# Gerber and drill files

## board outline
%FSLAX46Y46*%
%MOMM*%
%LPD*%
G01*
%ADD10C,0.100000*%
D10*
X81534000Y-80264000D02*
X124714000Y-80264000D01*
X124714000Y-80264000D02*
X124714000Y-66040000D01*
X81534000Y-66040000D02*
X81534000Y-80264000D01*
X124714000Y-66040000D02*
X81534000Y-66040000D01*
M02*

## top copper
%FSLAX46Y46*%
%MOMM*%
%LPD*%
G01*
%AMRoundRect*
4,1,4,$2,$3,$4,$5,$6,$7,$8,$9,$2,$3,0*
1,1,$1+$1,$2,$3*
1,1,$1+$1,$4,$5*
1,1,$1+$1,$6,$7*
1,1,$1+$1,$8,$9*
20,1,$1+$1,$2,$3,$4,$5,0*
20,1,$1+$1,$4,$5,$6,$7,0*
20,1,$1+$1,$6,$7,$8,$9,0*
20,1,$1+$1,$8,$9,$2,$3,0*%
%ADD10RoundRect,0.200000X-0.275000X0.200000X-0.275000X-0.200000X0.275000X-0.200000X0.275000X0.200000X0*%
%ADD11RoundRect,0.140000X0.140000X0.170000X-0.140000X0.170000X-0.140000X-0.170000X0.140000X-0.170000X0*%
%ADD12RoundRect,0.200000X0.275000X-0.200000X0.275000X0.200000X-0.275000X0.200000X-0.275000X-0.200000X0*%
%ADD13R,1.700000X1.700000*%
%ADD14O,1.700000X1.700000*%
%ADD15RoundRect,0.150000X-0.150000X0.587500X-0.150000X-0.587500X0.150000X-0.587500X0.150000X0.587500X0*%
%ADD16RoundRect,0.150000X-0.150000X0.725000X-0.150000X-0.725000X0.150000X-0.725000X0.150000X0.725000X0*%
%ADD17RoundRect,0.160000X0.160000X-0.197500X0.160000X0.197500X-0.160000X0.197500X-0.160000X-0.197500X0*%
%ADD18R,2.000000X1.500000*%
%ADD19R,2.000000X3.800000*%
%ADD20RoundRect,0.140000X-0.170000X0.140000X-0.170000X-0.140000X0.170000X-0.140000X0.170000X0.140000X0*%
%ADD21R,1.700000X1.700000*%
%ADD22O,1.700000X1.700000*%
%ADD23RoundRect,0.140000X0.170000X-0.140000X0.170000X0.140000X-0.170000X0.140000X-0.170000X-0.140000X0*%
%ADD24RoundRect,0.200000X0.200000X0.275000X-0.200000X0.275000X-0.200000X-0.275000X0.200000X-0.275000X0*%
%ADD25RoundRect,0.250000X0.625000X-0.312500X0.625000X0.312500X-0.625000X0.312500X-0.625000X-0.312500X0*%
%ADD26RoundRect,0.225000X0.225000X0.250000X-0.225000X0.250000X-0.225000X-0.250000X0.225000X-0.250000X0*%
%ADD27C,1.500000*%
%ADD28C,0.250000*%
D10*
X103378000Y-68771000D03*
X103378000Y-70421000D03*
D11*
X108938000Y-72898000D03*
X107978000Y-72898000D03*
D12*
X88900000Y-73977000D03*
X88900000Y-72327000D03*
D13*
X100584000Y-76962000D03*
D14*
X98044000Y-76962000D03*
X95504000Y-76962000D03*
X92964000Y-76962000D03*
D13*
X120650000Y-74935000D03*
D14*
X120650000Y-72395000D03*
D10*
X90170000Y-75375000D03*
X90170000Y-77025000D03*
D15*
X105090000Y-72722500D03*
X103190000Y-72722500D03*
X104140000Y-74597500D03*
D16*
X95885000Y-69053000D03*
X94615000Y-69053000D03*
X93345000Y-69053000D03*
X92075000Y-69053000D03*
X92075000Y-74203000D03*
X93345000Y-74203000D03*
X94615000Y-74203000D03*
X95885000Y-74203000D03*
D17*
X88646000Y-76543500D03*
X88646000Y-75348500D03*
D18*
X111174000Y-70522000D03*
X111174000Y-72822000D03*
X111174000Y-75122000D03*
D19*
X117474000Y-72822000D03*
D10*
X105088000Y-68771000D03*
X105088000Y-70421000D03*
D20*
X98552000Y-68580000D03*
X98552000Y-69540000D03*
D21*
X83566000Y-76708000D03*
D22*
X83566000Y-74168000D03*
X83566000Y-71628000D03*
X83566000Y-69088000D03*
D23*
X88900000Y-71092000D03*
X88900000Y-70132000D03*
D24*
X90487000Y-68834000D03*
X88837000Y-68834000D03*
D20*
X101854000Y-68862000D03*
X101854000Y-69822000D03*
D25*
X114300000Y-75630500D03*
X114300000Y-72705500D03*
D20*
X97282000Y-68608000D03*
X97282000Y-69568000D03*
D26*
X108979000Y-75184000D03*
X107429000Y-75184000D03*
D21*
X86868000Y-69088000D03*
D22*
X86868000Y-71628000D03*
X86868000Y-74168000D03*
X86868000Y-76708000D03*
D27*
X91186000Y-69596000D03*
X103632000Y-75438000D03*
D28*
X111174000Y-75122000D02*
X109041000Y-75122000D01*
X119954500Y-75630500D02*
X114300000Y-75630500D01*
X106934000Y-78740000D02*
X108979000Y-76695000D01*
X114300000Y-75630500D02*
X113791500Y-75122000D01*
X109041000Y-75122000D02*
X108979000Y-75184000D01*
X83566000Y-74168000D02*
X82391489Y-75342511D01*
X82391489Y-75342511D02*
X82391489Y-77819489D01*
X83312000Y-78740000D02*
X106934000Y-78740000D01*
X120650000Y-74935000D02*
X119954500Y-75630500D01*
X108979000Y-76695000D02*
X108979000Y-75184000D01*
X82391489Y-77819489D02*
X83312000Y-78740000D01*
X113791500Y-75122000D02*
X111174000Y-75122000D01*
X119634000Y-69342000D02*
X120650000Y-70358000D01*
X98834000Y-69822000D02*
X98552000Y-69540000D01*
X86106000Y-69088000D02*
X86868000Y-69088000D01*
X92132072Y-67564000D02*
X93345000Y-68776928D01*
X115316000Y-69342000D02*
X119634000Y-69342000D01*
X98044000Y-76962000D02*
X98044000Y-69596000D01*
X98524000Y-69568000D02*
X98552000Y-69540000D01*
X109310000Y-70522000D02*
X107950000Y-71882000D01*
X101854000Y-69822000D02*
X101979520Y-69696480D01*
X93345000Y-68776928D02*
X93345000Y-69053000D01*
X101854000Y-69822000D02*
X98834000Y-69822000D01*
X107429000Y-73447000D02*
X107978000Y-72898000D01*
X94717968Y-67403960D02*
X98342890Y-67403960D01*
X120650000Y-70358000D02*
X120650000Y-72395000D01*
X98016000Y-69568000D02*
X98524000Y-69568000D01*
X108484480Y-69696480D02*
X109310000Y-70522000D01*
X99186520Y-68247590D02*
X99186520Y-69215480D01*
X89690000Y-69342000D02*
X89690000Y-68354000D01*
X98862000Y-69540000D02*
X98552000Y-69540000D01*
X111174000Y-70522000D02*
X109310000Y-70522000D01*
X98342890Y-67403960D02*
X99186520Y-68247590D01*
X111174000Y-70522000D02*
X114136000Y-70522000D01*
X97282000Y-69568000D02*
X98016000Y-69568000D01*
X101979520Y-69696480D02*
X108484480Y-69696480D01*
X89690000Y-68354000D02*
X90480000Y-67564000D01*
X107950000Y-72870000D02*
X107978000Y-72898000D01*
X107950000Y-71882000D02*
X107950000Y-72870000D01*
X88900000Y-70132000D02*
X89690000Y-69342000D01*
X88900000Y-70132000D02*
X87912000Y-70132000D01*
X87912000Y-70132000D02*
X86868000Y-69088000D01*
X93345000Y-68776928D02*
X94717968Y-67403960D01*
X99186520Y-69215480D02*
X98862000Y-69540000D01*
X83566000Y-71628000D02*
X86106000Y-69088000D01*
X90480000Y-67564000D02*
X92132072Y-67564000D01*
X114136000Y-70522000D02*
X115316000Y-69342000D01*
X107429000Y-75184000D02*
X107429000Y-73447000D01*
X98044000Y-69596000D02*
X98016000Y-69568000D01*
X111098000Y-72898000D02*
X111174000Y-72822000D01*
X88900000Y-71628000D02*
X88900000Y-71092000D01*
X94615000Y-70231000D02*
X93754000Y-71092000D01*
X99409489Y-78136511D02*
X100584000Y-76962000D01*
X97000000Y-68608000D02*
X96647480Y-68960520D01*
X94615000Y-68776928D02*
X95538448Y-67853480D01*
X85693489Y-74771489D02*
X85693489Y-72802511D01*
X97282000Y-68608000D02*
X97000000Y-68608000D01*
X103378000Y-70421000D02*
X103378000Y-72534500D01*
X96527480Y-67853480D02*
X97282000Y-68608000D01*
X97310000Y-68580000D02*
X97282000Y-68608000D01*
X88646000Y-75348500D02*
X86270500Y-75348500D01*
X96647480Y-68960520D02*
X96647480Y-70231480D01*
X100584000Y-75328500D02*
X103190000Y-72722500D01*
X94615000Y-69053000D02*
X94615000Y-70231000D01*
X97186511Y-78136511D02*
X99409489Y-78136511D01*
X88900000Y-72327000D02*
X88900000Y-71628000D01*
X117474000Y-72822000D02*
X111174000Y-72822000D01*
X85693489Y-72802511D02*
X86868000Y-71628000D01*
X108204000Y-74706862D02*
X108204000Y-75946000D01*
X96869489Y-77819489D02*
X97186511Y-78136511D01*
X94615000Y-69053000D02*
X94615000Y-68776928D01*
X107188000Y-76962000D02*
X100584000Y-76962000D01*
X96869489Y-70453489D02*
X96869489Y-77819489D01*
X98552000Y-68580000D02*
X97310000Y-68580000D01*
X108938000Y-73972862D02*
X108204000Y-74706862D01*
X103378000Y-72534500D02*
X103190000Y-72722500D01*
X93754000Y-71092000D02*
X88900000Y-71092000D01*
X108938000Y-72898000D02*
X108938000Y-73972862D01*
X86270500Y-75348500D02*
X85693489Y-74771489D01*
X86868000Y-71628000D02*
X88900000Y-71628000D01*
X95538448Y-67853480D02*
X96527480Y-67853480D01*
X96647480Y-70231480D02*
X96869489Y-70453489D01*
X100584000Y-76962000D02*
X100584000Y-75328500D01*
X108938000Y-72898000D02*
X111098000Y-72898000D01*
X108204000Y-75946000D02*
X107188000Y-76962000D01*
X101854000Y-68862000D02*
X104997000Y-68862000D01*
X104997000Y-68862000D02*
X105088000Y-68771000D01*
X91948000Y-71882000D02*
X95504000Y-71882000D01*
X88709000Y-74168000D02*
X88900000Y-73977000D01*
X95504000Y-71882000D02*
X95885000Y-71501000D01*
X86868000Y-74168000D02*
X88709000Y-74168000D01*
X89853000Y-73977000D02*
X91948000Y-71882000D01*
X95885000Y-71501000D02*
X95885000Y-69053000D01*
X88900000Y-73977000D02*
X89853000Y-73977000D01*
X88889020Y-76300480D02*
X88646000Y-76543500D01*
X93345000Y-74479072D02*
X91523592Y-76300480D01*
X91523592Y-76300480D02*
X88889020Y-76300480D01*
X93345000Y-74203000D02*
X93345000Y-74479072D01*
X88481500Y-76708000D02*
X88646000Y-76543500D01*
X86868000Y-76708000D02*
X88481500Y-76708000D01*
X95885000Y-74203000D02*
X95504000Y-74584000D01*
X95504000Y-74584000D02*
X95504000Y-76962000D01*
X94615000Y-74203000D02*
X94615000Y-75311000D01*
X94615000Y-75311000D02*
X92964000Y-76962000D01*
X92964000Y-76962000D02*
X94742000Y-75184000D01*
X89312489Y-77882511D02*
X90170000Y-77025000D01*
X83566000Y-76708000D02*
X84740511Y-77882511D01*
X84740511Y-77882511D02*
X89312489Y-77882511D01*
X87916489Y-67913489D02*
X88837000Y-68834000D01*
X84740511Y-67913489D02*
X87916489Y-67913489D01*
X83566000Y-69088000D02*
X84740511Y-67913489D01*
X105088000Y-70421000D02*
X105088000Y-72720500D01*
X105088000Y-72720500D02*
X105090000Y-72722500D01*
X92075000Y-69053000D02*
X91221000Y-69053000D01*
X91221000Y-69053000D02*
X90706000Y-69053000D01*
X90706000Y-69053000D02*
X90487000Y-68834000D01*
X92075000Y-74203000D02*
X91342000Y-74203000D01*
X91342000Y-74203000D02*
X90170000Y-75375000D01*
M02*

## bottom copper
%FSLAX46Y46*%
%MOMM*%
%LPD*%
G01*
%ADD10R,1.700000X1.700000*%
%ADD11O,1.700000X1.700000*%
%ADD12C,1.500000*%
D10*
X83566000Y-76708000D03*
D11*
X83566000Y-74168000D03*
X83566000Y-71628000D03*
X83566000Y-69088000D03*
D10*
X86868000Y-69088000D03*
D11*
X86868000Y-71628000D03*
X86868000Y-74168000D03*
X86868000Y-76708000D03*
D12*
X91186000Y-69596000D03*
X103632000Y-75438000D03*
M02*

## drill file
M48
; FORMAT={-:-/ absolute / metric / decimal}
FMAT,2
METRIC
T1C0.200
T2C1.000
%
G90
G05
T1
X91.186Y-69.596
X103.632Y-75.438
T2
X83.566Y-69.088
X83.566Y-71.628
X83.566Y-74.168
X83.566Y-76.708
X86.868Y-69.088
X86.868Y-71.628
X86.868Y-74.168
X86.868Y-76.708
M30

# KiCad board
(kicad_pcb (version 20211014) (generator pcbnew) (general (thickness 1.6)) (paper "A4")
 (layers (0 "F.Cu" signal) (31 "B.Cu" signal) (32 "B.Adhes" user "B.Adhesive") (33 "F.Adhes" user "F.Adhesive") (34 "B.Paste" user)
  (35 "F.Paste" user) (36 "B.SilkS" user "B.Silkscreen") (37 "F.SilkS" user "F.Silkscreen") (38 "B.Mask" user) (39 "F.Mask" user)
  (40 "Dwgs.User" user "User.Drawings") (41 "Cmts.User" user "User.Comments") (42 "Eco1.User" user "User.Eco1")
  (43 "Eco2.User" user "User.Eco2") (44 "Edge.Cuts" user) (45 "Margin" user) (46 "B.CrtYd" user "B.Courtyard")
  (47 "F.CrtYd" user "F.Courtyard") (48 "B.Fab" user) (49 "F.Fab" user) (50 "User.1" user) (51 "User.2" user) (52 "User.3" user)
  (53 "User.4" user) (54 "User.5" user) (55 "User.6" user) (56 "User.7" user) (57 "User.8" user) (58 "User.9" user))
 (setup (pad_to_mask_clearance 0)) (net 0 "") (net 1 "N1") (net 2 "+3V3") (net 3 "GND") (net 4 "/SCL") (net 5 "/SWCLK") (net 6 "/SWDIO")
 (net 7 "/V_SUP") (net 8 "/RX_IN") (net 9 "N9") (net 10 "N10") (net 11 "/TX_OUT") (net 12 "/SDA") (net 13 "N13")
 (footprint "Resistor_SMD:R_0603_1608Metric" (layer "F.Cu") (at 103.378 69.596 -90)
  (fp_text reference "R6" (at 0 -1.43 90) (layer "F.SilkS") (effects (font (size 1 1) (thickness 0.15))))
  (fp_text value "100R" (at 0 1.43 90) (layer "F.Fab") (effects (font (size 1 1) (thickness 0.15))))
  (pad "1" smd roundrect locked (at -0.825 0 270) (size 0.8 0.95) (layers "F.Cu" "F.Paste" "F.Mask") (roundrect_rratio 0.25) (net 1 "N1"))
  (pad "2" smd roundrect locked (at 0.825 0 270) (size 0.8 0.95) (layers "F.Cu" "F.Paste" "F.Mask") (roundrect_rratio 0.25) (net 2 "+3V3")))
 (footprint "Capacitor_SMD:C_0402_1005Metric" (layer "F.Cu") (at 108.458 72.898 180)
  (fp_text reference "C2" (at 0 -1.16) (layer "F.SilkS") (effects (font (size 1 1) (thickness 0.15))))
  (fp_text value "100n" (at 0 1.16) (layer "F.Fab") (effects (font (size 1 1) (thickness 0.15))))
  (pad "1" smd roundrect locked (at -0.48 0 180) (size 0.56 0.62) (layers "F.Cu" "F.Paste" "F.Mask") (roundrect_rratio 0.25) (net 2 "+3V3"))
  (pad "2" smd roundrect locked (at 0.48 0 180) (size 0.56 0.62) (layers "F.Cu" "F.Paste" "F.Mask") (roundrect_rratio 0.25) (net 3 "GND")))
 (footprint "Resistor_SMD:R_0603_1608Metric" (layer "F.Cu") (at 88.9 73.152 90)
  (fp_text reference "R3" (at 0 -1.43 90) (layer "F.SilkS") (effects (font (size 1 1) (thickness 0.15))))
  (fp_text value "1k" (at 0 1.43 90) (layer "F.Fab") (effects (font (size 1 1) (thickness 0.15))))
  (pad "1" smd roundrect locked (at -0.825 0 90) (size 0.8 0.95) (layers "F.Cu" "F.Paste" "F.Mask") (roundrect_rratio 0.25) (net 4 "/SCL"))
  (pad "2" smd roundrect locked (at 0.825 0 90) (size 0.8 0.95) (layers "F.Cu" "F.Paste" "F.Mask") (roundrect_rratio 0.25) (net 2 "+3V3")))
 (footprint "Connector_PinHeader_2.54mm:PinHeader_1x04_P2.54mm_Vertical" (layer "F.Cu") (at 100.584 76.962 -90)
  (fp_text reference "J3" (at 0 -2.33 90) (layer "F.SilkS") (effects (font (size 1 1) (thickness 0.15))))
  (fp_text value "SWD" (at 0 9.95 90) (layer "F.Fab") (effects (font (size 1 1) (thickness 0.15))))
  (pad "1" smd rect locked (at 0 0 270) (size 1.7 1.7) (layers "F.Cu" "F.Paste" "F.Mask") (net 2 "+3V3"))
  (pad "2" smd oval locked (at 0 2.54 270) (size 1.7 1.7) (layers "F.Cu" "F.Paste" "F.Mask") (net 3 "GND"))
  (pad "3" smd oval locked (at 0 5.08 270) (size 1.7 1.7) (layers "F.Cu" "F.Paste" "F.Mask") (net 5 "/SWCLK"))
  (pad "4" smd oval locked (at 0 7.62 270) (size 1.7 1.7) (layers "F.Cu" "F.Paste" "F.Mask") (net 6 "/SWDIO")))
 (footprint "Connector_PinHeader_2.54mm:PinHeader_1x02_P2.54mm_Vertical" (layer "F.Cu") (at 120.65 74.935 180)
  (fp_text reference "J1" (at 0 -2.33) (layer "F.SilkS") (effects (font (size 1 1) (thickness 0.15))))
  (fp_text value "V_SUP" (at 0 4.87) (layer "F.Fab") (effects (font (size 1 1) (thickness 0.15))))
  (pad "1" smd rect locked (at 0 0 180) (size 1.7 1.7) (layers "F.Cu" "F.Paste" "F.Mask") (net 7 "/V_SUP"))
  (pad "2" smd oval locked (at 0 2.54 180) (size 1.7 1.7) (layers "F.Cu" "F.Paste" "F.Mask") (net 3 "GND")))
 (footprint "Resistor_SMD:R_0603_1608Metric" (layer "F.Cu") (at 90.17 76.2 -90)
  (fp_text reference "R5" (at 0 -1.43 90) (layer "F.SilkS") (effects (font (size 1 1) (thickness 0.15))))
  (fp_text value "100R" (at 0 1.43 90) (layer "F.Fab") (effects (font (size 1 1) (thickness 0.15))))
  (pad "1" smd roundrect locked (at -0.825 0 270) (size 0.8 0.95) (layers "F.Cu" "F.Paste" "F.Mask") (roundrect_rratio 0.25)
   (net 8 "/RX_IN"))
  (pad "2" smd roundrect locked (at 0.825 0 270) (size 0.8 0.95) (layers "F.Cu" "F.Paste" "F.Mask") (roundrect_rratio 0.25) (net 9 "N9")))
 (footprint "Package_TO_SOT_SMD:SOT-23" (layer "F.Cu") (at 104.14 73.66 -90)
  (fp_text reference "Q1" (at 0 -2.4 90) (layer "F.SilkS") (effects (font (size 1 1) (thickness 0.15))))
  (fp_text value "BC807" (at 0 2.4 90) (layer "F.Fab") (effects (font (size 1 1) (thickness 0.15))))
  (pad "1" smd roundrect locked (at -0.9375 -0.95 270) (size 1.475 0.6) (layers "F.Cu" "F.Paste" "F.Mask") (roundrect_rratio 0.25)
   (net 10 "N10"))
  (pad "2" smd roundrect locked (at -0.9375 0.95 270) (size 1.475 0.6) (layers "F.Cu" "F.Paste" "F.Mask") (roundrect_rratio 0.25)
   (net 2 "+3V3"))
  (pad "3" smd roundrect locked (at 0.9375 0 270) (size 1.475 0.6) (layers "F.Cu" "F.Paste" "F.Mask") (roundrect_rratio 0.25)
   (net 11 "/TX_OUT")))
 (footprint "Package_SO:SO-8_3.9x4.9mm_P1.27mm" (layer "F.Cu") (at 93.98 71.628 -90)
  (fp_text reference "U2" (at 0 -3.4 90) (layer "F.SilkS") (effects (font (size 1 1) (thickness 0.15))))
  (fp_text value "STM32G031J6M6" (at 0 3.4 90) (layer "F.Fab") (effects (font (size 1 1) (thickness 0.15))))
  (pad "1" smd roundrect locked (at -2.575 -1.905 270) (size 1.75 0.6) (layers "F.Cu" "F.Paste" "F.Mask") (roundrect_rratio 0.25)
   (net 4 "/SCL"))
  (pad "2" smd roundrect locked (at -2.575 -0.635 270) (size 1.75 0.6) (layers "F.Cu" "F.Paste" "F.Mask") (roundrect_rratio 0.25)
   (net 2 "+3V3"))
  (pad "3" smd roundrect locked (at -2.575 0.635 270) (size 1.75 0.6) (layers "F.Cu" "F.Paste" "F.Mask") (roundrect_rratio 0.25)
   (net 3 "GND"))
  (pad "4" smd roundrect locked (at -2.575 1.905 270) (size 1.75 0.6) (layers "F.Cu" "F.Paste" "F.Mask") (roundrect_rratio 0.25)
   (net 11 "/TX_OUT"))
  (pad "5" smd roundrect locked (at 2.575 1.905 270) (size 1.75 0.6) (layers "F.Cu" "F.Paste" "F.Mask") (roundrect_rratio 0.25)
   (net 8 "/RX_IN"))
  (pad "6" smd roundrect locked (at 2.575 0.635 270) (size 1.75 0.6) (layers "F.Cu" "F.Paste" "F.Mask") (roundrect_rratio 0.25)
   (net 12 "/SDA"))
  (pad "7" smd roundrect locked (at 2.575 -0.635 270) (size 1.75 0.6) (layers "F.Cu" "F.Paste" "F.Mask") (roundrect_rratio 0.25)
   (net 6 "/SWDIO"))
  (pad "8" smd roundrect locked (at 2.575 -1.905 270) (size 1.75 0.6) (layers "F.Cu" "F.Paste" "F.Mask") (roundrect_rratio 0.25)
   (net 5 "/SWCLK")))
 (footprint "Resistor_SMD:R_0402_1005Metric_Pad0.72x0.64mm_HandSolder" (layer "F.Cu") (at 88.646 75.946 90)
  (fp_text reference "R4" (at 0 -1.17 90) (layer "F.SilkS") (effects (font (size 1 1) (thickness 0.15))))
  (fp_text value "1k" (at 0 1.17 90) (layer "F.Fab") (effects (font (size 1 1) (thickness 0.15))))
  (pad "1" smd roundrect locked (at -0.5975 0 90) (size 0.715 0.64) (layers "F.Cu" "F.Paste" "F.Mask") (roundrect_rratio 0.25)
   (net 12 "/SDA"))
  (pad "2" smd roundrect locked (at 0.5975 0 90) (size 0.715 0.64) (layers "F.Cu" "F.Paste" "F.Mask") (roundrect_rratio 0.25) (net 2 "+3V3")))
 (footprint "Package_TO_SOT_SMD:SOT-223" (layer "F.Cu") (at 114.324 72.822)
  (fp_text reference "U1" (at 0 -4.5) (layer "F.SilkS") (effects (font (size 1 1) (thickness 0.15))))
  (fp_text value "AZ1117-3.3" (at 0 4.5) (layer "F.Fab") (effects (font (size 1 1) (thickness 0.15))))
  (pad "1" smd rect locked (at -3.15 -2.3) (size 2 1.5) (layers "F.Cu" "F.Paste" "F.Mask") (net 3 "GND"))
  (pad "2" smd rect locked (at -3.15 0) (size 2 1.5) (layers "F.Cu" "F.Paste" "F.Mask") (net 2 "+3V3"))
  (pad "3" smd rect locked (at -3.15 2.3) (size 2 1.5) (layers "F.Cu" "F.Paste" "F.Mask") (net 7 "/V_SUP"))
  (pad "4" smd rect locked (at 3.15 0) (size 2 3.8) (layers "F.Cu" "F.Paste" "F.Mask") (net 2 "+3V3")))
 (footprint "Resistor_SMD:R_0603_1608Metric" (layer "F.Cu") (at 105.088 69.596 -90)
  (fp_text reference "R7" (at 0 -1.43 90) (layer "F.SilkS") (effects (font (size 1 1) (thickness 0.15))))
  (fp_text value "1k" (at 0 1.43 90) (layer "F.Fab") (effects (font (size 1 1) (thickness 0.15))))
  (pad "1" smd roundrect locked (at -0.825 0 270) (size 0.8 0.95) (layers "F.Cu" "F.Paste" "F.Mask") (roundrect_rratio 0.25) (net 1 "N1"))
  (pad "2" smd roundrect locked (at 0.825 0 270) (size 0.8 0.95) (layers "F.Cu" "F.Paste" "F.Mask") (roundrect_rratio 0.25) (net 10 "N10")))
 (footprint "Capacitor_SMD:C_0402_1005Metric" (layer "F.Cu") (at 98.552 69.06 -90)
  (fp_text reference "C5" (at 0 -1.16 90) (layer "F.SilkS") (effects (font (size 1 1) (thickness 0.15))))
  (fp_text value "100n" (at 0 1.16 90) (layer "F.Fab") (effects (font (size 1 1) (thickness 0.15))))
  (pad "1" smd roundrect locked (at -0.48 0 270) (size 0.56 0.62) (layers "F.Cu" "F.Paste" "F.Mask") (roundrect_rratio 0.25) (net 2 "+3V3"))
  (pad "2" smd roundrect locked (at 0.48 0 270) (size 0.56 0.62) (layers "F.Cu" "F.Paste" "F.Mask") (roundrect_rratio 0.25) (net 3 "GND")))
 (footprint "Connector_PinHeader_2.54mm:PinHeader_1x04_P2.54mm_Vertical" (layer "F.Cu") (at 83.566 76.708 180)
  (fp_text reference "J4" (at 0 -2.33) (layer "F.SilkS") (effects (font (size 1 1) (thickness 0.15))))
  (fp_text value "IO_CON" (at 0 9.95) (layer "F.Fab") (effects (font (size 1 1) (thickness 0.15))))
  (pad "1" thru_hole rect locked (at 0 0 180) (size 1.7 1.7) (drill 1) (layers *.Cu *.Mask) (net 9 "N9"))
  (pad "2" thru_hole oval locked (at 0 2.54 180) (size 1.7 1.7) (drill 1) (layers *.Cu *.Mask) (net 7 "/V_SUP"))
  (pad "3" thru_hole oval locked (at 0 5.08 180) (size 1.7 1.7) (drill 1) (layers *.Cu *.Mask) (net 3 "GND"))
  (pad "4" thru_hole oval locked (at 0 7.62 180) (size 1.7 1.7) (drill 1) (layers *.Cu *.Mask) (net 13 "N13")))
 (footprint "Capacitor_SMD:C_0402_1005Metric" (layer "F.Cu") (at 88.9 70.612 90)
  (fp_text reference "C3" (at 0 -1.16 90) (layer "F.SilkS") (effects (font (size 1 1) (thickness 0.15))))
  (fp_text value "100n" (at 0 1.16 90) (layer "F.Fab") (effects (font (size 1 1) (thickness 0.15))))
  (pad "1" smd roundrect locked (at -0.48 0 90) (size 0.56 0.62) (layers "F.Cu" "F.Paste" "F.Mask") (roundrect_rratio 0.25) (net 2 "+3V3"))
  (pad "2" smd roundrect locked (at 0.48 0 90) (size 0.56 0.62) (layers "F.Cu" "F.Paste" "F.Mask") (roundrect_rratio 0.25) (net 3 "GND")))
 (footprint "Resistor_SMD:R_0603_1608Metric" (layer "F.Cu") (at 89.662 68.834 180)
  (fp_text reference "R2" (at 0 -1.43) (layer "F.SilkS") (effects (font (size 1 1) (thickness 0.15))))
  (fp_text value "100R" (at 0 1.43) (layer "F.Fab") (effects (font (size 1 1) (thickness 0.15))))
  (pad "1" smd roundrect locked (at -0.825 0 180) (size 0.8 0.95) (layers "F.Cu" "F.Paste" "F.Mask") (roundrect_rratio 0.25)
   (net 11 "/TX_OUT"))
  (pad "2" smd roundrect locked (at 0.825 0 180) (size 0.8 0.95) (layers "F.Cu" "F.Paste" "F.Mask") (roundrect_rratio 0.25) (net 13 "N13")))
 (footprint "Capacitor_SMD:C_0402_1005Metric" (layer "F.Cu") (at 101.854 69.342 -90)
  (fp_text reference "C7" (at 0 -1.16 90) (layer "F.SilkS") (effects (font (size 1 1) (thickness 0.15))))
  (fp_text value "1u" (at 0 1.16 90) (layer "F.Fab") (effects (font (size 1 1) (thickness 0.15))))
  (pad "1" smd roundrect locked (at -0.48 0 270) (size 0.56 0.62) (layers "F.Cu" "F.Paste" "F.Mask") (roundrect_rratio 0.25) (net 1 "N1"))
  (pad "2" smd roundrect locked (at 0.48 0 270) (size 0.56 0.62) (layers "F.Cu" "F.Paste" "F.Mask") (roundrect_rratio 0.25) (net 3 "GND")))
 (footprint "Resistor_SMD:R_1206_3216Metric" (layer "F.Cu") (at 114.3 74.168 90)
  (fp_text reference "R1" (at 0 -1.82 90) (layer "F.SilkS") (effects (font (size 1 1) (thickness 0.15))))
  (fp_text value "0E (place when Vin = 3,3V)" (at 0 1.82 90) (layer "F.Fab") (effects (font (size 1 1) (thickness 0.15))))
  (pad "1" smd roundrect locked (at -1.4625 0 90) (size 1.125 1.75) (layers "F.Cu" "F.Paste" "F.Mask") (roundrect_rratio 0.222222)
   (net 7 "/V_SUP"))
  (pad "2" smd roundrect locked (at 1.4625 0 90) (size 1.125 1.75) (layers "F.Cu" "F.Paste" "F.Mask") (roundrect_rratio 0.222222)
   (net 2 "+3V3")))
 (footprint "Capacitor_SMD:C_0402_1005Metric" (layer "F.Cu") (at 97.282 69.088 -90)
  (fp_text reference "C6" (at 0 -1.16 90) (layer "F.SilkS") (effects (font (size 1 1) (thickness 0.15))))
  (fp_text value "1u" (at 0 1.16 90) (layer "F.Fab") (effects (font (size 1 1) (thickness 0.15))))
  (pad "1" smd roundrect locked (at -0.48 0 270) (size 0.56 0.62) (layers "F.Cu" "F.Paste" "F.Mask") (roundrect_rratio 0.25) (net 2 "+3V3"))
  (pad "2" smd roundrect locked (at 0.48 0 270) (size 0.56 0.62) (layers "F.Cu" "F.Paste" "F.Mask") (roundrect_rratio 0.25) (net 3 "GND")))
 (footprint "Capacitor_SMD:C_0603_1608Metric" (layer "F.Cu") (at 108.204 75.184 180)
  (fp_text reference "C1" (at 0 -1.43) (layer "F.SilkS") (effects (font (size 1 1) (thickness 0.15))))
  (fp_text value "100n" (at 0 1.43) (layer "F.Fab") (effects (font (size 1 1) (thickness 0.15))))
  (pad "1" smd roundrect locked (at -0.775 0 180) (size 0.9 0.95) (layers "F.Cu" "F.Paste" "F.Mask") (roundrect_rratio 0.25)
   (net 7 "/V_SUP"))
  (pad "2" smd roundrect locked (at 0.775 0 180) (size 0.9 0.95) (layers "F.Cu" "F.Paste" "F.Mask") (roundrect_rratio 0.25) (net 3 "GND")))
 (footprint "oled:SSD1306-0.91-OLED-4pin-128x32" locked (layer "B.Cu") (at 123.368 66.898 180)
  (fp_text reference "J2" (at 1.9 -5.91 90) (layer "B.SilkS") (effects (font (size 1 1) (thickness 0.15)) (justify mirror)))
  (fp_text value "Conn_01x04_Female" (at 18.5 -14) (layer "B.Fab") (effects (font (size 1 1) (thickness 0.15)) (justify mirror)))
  (pad "1" thru_hole rect locked (at 36.5 -2.19 180) (size 1.7 1.7) (drill 1) (layers *.Cu *.Mask) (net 3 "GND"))
  (pad "2" thru_hole oval locked (at 36.5 -4.73 180) (size 1.7 1.7) (drill 1) (layers *.Cu *.Mask) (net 2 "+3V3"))
  (pad "3" thru_hole oval locked (at 36.5 -7.27 180) (size 1.7 1.7) (drill 1) (layers *.Cu *.Mask) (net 4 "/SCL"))
  (pad "4" thru_hole oval locked (at 36.5 -9.81 180) (size 1.7 1.7) (drill 1) (layers *.Cu *.Mask) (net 12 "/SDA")))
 (gr_line (start 81.534 80.264) (end 124.714 80.264) (layer "Edge.Cuts") (width 0.1))
 (gr_line (start 124.714 80.264) (end 124.714 66.04) (layer "Edge.Cuts") (width 0.1))
 (gr_line (start 81.534 66.04) (end 81.534 80.264) (layer "Edge.Cuts") (width 0.1))
 (gr_line (start 124.714 66.04) (end 81.534 66.04) (layer "Edge.Cuts") (width 0.1))
 (segment (start 111.174 75.122) (end 109.041 75.122) (width 0.25) (layer "F.Cu") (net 7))
 (segment (start 119.9545 75.6305) (end 114.3 75.6305) (width 0.25) (layer "F.Cu") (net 7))
 (segment (start 106.934 78.74) (end 108.979 76.695) (width 0.25) (layer "F.Cu") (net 7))
 (segment (start 114.3 75.6305) (end 113.7915 75.122) (width 0.25) (layer "F.Cu") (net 7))
 (segment (start 109.041 75.122) (end 108.979 75.184) (width 0.25) (layer "F.Cu") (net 7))
 (segment (start 83.566 74.168) (end 82.391489 75.342511) (width 0.25) (layer "F.Cu") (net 7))
 (segment (start 82.391489 75.342511) (end 82.391489 77.819489) (width 0.25) (layer "F.Cu") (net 7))
 (segment (start 83.312 78.74) (end 106.934 78.74) (width 0.25) (layer "F.Cu") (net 7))
 (segment (start 120.65 74.935) (end 119.9545 75.6305) (width 0.25) (layer "F.Cu") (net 7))
 (segment (start 108.979 76.695) (end 108.979 75.184) (width 0.25) (layer "F.Cu") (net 7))
 (segment (start 82.391489 77.819489) (end 83.312 78.74) (width 0.25) (layer "F.Cu") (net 7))
 (segment (start 113.7915 75.122) (end 111.174 75.122) (width 0.25) (layer "F.Cu") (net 7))
 (segment (start 119.634 69.342) (end 120.65 70.358) (width 0.25) (layer "F.Cu") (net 3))
 (segment (start 98.834 69.822) (end 98.552 69.54) (width 0.25) (layer "F.Cu") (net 3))
 (segment (start 86.106 69.088) (end 86.868 69.088) (width 0.25) (layer "F.Cu") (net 3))
 (segment (start 92.132072 67.564) (end 93.345 68.776928) (width 0.25) (layer "F.Cu") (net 3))
 (segment (start 115.316 69.342) (end 119.634 69.342) (width 0.25) (layer "F.Cu") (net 3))
 (segment (start 98.044 76.962) (end 98.044 69.596) (width 0.25) (layer "F.Cu") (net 3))
 (segment (start 98.524 69.568) (end 98.552 69.54) (width 0.25) (layer "F.Cu") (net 3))
 (segment (start 109.31 70.522) (end 107.95 71.882) (width 0.25) (layer "F.Cu") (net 3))
 (segment (start 101.854 69.822) (end 101.97952 69.69648) (width 0.25) (layer "F.Cu") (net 3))
 (segment (start 93.345 68.776928) (end 93.345 69.053) (width 0.25) (layer "F.Cu") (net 3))
 (segment (start 101.854 69.822) (end 98.834 69.822) (width 0.25) (layer "F.Cu") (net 3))
 (segment (start 107.429 73.447) (end 107.978 72.898) (width 0.25) (layer "F.Cu") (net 3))
 (segment (start 94.717968 67.40396) (end 98.34289 67.40396) (width 0.25) (layer "F.Cu") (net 3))
 (segment (start 120.65 70.358) (end 120.65 72.395) (width 0.25) (layer "F.Cu") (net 3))
 (segment (start 98.016 69.568) (end 98.524 69.568) (width 0.25) (layer "F.Cu") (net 3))
 (segment (start 108.48448 69.69648) (end 109.31 70.522) (width 0.25) (layer "F.Cu") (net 3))
 (segment (start 99.18652 68.24759) (end 99.18652 69.21548) (width 0.25) (layer "F.Cu") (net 3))
 (segment (start 89.69 69.342) (end 89.69 68.354) (width 0.25) (layer "F.Cu") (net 3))
 (segment (start 98.862 69.54) (end 98.552 69.54) (width 0.25) (layer "F.Cu") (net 3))
 (segment (start 111.174 70.522) (end 109.31 70.522) (width 0.25) (layer "F.Cu") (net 3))
 (segment (start 98.34289 67.40396) (end 99.18652 68.24759) (width 0.25) (layer "F.Cu") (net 3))
 (segment (start 111.174 70.522) (end 114.136 70.522) (width 0.25) (layer "F.Cu") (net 3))
 (segment (start 97.282 69.568) (end 98.016 69.568) (width 0.25) (layer "F.Cu") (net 3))
 (segment (start 101.97952 69.69648) (end 108.48448 69.69648) (width 0.25) (layer "F.Cu") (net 3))
 (segment (start 89.69 68.354) (end 90.48 67.564) (width 0.25) (layer "F.Cu") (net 3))
 (segment (start 107.95 72.87) (end 107.978 72.898) (width 0.25) (layer "F.Cu") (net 3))
 (segment (start 107.95 71.882) (end 107.95 72.87) (width 0.25) (layer "F.Cu") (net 3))
 (segment (start 88.9 70.132) (end 89.69 69.342) (width 0.25) (layer "F.Cu") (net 3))
 (segment (start 88.9 70.132) (end 87.912 70.132) (width 0.25) (layer "F.Cu") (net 3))
 (segment (start 87.912 70.132) (end 86.868 69.088) (width 0.25) (layer "F.Cu") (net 3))
 (segment (start 93.345 68.776928) (end 94.717968 67.40396) (width 0.25) (layer "F.Cu") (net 3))
 (segment (start 99.18652 69.21548) (end 98.862 69.54) (width 0.25) (layer "F.Cu") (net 3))
 (segment (start 83.566 71.628) (end 86.106 69.088) (width 0.25) (layer "F.Cu") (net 3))
 (segment (start 90.48 67.564) (end 92.132072 67.564) (width 0.25) (layer "F.Cu") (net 3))
 (segment (start 114.136 70.522) (end 115.316 69.342) (width 0.25) (layer "F.Cu") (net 3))
 (segment (start 107.429 75.184) (end 107.429 73.447) (width 0.25) (layer "F.Cu") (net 3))
 (segment (start 98.044 69.596) (end 98.016 69.568) (width 0.25) (layer "F.Cu") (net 3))
 (segment (start 111.098 72.898) (end 111.174 72.822) (width 0.25) (layer "F.Cu") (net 2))
 (segment (start 88.9 71.628) (end 88.9 71.092) (width 0.25) (layer "F.Cu") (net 2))
 (segment (start 94.615 70.231) (end 93.754 71.092) (width 0.25) (layer "F.Cu") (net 2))
 (segment (start 99.409489 78.136511) (end 100.584 76.962) (width 0.25) (layer "F.Cu") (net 2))
 (segment (start 97 68.608) (end 96.64748 68.96052) (width 0.25) (layer "F.Cu") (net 2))
 (segment (start 94.615 68.776928) (end 95.538448 67.85348) (width 0.25) (layer "F.Cu") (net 2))
 (segment (start 85.693489 74.771489) (end 85.693489 72.802511) (width 0.25) (layer "F.Cu") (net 2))
 (segment (start 97.282 68.608) (end 97 68.608) (width 0.25) (layer "F.Cu") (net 2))
 (segment (start 103.378 70.421) (end 103.378 72.5345) (width 0.25) (layer "F.Cu") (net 2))
 (segment (start 96.52748 67.85348) (end 97.282 68.608) (width 0.25) (layer "F.Cu") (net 2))
 (segment (start 97.31 68.58) (end 97.282 68.608) (width 0.25) (layer "F.Cu") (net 2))
 (segment (start 88.646 75.3485) (end 86.2705 75.3485) (width 0.25) (layer "F.Cu") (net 2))
 (segment (start 96.64748 68.96052) (end 96.64748 70.23148) (width 0.25) (layer "F.Cu") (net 2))
 (segment (start 100.584 75.3285) (end 103.19 72.7225) (width 0.25) (layer "F.Cu") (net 2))
 (segment (start 94.615 69.053) (end 94.615 70.231) (width 0.25) (layer "F.Cu") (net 2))
 (segment (start 97.186511 78.136511) (end 99.409489 78.136511) (width 0.25) (layer "F.Cu") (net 2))
 (segment (start 88.9 72.327) (end 88.9 71.628) (width 0.25) (layer "F.Cu") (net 2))
 (segment (start 117.474 72.822) (end 111.174 72.822) (width 0.25) (layer "F.Cu") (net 2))
 (segment (start 85.693489 72.802511) (end 86.868 71.628) (width 0.25) (layer "F.Cu") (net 2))
 (segment (start 108.204 74.706862) (end 108.204 75.946) (width 0.25) (layer "F.Cu") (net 2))
 (segment (start 96.869489 77.819489) (end 97.186511 78.136511) (width 0.25) (layer "F.Cu") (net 2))
 (segment (start 94.615 69.053) (end 94.615 68.776928) (width 0.25) (layer "F.Cu") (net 2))
 (segment (start 107.188 76.962) (end 100.584 76.962) (width 0.25) (layer "F.Cu") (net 2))
 (segment (start 96.869489 70.453489) (end 96.869489 77.819489) (width 0.25) (layer "F.Cu") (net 2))
 (segment (start 98.552 68.58) (end 97.31 68.58) (width 0.25) (layer "F.Cu") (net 2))
 (segment (start 108.938 73.972862) (end 108.204 74.706862) (width 0.25) (layer "F.Cu") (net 2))
 (segment (start 103.378 72.5345) (end 103.19 72.7225) (width 0.25) (layer "F.Cu") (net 2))
 (segment (start 93.754 71.092) (end 88.9 71.092) (width 0.25) (layer "F.Cu") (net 2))
 (segment (start 108.938 72.898) (end 108.938 73.972862) (width 0.25) (layer "F.Cu") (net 2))
 (segment (start 86.2705 75.3485) (end 85.693489 74.771489) (width 0.25) (layer "F.Cu") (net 2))
 (segment (start 86.868 71.628) (end 88.9 71.628) (width 0.25) (layer "F.Cu") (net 2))
 (segment (start 95.538448 67.85348) (end 96.52748 67.85348) (width 0.25) (layer "F.Cu") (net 2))
 (segment (start 96.64748 70.23148) (end 96.869489 70.453489) (width 0.25) (layer "F.Cu") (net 2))
 (segment (start 100.584 76.962) (end 100.584 75.3285) (width 0.25) (layer "F.Cu") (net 2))
 (segment (start 108.938 72.898) (end 111.098 72.898) (width 0.25) (layer "F.Cu") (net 2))
 (segment (start 108.204 75.946) (end 107.188 76.962) (width 0.25) (layer "F.Cu") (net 2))
 (segment (start 101.854 68.862) (end 104.997 68.862) (width 0.25) (layer "F.Cu") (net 1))
 (segment (start 104.997 68.862) (end 105.088 68.771) (width 0.25) (layer "F.Cu") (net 1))
 (segment (start 91.948 71.882) (end 95.504 71.882) (width 0.25) (layer "F.Cu") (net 4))
 (segment (start 88.709 74.168) (end 88.9 73.977) (width 0.25) (layer "F.Cu") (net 4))
 (segment (start 95.504 71.882) (end 95.885 71.501) (width 0.25) (layer "F.Cu") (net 4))
 (segment (start 86.868 74.168) (end 88.709 74.168) (width 0.25) (layer "F.Cu") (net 4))
 (segment (start 89.853 73.977) (end 91.948 71.882) (width 0.25) (layer "F.Cu") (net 4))
 (segment (start 95.885 71.501) (end 95.885 69.053) (width 0.25) (layer "F.Cu") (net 4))
 (segment (start 88.9 73.977) (end 89.853 73.977) (width 0.25) (layer "F.Cu") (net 4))
 (segment (start 88.88902 76.30048) (end 88.646 76.5435) (width 0.25) (layer "F.Cu") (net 12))
 (segment (start 93.345 74.479072) (end 91.523592 76.30048) (width 0.25) (layer "F.Cu") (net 12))
 (segment (start 91.523592 76.30048) (end 88.88902 76.30048) (width 0.25) (layer "F.Cu") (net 12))
 (segment (start 93.345 74.203) (end 93.345 74.479072) (width 0.25) (layer "F.Cu") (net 12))
 (segment (start 88.4815 76.708) (end 88.646 76.5435) (width 0.25) (layer "F.Cu") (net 12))
 (segment (start 86.868 76.708) (end 88.4815 76.708) (width 0.25) (layer "F.Cu") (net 12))
 (segment (start 95.885 74.203) (end 95.504 74.584) (width 0.25) (layer "F.Cu") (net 5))
 (segment (start 95.504 74.584) (end 95.504 76.962) (width 0.25) (layer "F.Cu") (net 5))
 (segment (start 94.615 74.203) (end 94.615 75.311) (width 0.25) (layer "F.Cu") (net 6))
 (segment (start 94.615 75.311) (end 92.964 76.962) (width 0.25) (layer "F.Cu") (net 6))
 (segment (start 92.964 76.962) (end 94.742 75.184) (width 0.25) (layer "F.Cu") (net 6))
 (segment (start 89.312489 77.882511) (end 90.17 77.025) (width 0.25) (layer "F.Cu") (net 9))
 (segment (start 83.566 76.708) (end 84.740511 77.882511) (width 0.25) (layer "F.Cu") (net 9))
 (segment (start 84.740511 77.882511) (end 89.312489 77.882511) (width 0.25) (layer "F.Cu") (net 9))
 (segment (start 87.916489 67.913489) (end 88.837 68.834) (width 0.25) (layer "F.Cu") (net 13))
 (segment (start 84.740511 67.913489) (end 87.916489 67.913489) (width 0.25) (layer "F.Cu") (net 13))
 (segment (start 83.566 69.088) (end 84.740511 67.913489) (width 0.25) (layer "F.Cu") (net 13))
 (segment (start 105.088 70.421) (end 105.088 72.7205) (width 0.25) (layer "F.Cu") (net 10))
 (segment (start 105.088 72.7205) (end 105.09 72.7225) (width 0.25) (layer "F.Cu") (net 10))
 (segment (start 92.075 69.053) (end 91.221 69.053) (width 0.25) (layer "F.Cu") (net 11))
 (segment (start 91.221 69.053) (end 90.706 69.053) (width 0.25) (layer "F.Cu") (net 11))
 (segment (start 90.706 69.053) (end 90.487 68.834) (width 0.25) (layer "F.Cu") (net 11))
 (via (at 91.186 69.596) (size 1.5) (drill 0.2) (layers "F.Cu" "B.Cu") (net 11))
 (via (at 103.632 75.438) (size 1.5) (drill 0.2) (layers "F.Cu" "B.Cu") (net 11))
 (segment (start 92.075 74.203) (end 91.342 74.203) (width 0.25) (layer "F.Cu") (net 8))
 (segment (start 91.342 74.203) (end 90.17 75.375) (width 0.25) (layer "F.Cu") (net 8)))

